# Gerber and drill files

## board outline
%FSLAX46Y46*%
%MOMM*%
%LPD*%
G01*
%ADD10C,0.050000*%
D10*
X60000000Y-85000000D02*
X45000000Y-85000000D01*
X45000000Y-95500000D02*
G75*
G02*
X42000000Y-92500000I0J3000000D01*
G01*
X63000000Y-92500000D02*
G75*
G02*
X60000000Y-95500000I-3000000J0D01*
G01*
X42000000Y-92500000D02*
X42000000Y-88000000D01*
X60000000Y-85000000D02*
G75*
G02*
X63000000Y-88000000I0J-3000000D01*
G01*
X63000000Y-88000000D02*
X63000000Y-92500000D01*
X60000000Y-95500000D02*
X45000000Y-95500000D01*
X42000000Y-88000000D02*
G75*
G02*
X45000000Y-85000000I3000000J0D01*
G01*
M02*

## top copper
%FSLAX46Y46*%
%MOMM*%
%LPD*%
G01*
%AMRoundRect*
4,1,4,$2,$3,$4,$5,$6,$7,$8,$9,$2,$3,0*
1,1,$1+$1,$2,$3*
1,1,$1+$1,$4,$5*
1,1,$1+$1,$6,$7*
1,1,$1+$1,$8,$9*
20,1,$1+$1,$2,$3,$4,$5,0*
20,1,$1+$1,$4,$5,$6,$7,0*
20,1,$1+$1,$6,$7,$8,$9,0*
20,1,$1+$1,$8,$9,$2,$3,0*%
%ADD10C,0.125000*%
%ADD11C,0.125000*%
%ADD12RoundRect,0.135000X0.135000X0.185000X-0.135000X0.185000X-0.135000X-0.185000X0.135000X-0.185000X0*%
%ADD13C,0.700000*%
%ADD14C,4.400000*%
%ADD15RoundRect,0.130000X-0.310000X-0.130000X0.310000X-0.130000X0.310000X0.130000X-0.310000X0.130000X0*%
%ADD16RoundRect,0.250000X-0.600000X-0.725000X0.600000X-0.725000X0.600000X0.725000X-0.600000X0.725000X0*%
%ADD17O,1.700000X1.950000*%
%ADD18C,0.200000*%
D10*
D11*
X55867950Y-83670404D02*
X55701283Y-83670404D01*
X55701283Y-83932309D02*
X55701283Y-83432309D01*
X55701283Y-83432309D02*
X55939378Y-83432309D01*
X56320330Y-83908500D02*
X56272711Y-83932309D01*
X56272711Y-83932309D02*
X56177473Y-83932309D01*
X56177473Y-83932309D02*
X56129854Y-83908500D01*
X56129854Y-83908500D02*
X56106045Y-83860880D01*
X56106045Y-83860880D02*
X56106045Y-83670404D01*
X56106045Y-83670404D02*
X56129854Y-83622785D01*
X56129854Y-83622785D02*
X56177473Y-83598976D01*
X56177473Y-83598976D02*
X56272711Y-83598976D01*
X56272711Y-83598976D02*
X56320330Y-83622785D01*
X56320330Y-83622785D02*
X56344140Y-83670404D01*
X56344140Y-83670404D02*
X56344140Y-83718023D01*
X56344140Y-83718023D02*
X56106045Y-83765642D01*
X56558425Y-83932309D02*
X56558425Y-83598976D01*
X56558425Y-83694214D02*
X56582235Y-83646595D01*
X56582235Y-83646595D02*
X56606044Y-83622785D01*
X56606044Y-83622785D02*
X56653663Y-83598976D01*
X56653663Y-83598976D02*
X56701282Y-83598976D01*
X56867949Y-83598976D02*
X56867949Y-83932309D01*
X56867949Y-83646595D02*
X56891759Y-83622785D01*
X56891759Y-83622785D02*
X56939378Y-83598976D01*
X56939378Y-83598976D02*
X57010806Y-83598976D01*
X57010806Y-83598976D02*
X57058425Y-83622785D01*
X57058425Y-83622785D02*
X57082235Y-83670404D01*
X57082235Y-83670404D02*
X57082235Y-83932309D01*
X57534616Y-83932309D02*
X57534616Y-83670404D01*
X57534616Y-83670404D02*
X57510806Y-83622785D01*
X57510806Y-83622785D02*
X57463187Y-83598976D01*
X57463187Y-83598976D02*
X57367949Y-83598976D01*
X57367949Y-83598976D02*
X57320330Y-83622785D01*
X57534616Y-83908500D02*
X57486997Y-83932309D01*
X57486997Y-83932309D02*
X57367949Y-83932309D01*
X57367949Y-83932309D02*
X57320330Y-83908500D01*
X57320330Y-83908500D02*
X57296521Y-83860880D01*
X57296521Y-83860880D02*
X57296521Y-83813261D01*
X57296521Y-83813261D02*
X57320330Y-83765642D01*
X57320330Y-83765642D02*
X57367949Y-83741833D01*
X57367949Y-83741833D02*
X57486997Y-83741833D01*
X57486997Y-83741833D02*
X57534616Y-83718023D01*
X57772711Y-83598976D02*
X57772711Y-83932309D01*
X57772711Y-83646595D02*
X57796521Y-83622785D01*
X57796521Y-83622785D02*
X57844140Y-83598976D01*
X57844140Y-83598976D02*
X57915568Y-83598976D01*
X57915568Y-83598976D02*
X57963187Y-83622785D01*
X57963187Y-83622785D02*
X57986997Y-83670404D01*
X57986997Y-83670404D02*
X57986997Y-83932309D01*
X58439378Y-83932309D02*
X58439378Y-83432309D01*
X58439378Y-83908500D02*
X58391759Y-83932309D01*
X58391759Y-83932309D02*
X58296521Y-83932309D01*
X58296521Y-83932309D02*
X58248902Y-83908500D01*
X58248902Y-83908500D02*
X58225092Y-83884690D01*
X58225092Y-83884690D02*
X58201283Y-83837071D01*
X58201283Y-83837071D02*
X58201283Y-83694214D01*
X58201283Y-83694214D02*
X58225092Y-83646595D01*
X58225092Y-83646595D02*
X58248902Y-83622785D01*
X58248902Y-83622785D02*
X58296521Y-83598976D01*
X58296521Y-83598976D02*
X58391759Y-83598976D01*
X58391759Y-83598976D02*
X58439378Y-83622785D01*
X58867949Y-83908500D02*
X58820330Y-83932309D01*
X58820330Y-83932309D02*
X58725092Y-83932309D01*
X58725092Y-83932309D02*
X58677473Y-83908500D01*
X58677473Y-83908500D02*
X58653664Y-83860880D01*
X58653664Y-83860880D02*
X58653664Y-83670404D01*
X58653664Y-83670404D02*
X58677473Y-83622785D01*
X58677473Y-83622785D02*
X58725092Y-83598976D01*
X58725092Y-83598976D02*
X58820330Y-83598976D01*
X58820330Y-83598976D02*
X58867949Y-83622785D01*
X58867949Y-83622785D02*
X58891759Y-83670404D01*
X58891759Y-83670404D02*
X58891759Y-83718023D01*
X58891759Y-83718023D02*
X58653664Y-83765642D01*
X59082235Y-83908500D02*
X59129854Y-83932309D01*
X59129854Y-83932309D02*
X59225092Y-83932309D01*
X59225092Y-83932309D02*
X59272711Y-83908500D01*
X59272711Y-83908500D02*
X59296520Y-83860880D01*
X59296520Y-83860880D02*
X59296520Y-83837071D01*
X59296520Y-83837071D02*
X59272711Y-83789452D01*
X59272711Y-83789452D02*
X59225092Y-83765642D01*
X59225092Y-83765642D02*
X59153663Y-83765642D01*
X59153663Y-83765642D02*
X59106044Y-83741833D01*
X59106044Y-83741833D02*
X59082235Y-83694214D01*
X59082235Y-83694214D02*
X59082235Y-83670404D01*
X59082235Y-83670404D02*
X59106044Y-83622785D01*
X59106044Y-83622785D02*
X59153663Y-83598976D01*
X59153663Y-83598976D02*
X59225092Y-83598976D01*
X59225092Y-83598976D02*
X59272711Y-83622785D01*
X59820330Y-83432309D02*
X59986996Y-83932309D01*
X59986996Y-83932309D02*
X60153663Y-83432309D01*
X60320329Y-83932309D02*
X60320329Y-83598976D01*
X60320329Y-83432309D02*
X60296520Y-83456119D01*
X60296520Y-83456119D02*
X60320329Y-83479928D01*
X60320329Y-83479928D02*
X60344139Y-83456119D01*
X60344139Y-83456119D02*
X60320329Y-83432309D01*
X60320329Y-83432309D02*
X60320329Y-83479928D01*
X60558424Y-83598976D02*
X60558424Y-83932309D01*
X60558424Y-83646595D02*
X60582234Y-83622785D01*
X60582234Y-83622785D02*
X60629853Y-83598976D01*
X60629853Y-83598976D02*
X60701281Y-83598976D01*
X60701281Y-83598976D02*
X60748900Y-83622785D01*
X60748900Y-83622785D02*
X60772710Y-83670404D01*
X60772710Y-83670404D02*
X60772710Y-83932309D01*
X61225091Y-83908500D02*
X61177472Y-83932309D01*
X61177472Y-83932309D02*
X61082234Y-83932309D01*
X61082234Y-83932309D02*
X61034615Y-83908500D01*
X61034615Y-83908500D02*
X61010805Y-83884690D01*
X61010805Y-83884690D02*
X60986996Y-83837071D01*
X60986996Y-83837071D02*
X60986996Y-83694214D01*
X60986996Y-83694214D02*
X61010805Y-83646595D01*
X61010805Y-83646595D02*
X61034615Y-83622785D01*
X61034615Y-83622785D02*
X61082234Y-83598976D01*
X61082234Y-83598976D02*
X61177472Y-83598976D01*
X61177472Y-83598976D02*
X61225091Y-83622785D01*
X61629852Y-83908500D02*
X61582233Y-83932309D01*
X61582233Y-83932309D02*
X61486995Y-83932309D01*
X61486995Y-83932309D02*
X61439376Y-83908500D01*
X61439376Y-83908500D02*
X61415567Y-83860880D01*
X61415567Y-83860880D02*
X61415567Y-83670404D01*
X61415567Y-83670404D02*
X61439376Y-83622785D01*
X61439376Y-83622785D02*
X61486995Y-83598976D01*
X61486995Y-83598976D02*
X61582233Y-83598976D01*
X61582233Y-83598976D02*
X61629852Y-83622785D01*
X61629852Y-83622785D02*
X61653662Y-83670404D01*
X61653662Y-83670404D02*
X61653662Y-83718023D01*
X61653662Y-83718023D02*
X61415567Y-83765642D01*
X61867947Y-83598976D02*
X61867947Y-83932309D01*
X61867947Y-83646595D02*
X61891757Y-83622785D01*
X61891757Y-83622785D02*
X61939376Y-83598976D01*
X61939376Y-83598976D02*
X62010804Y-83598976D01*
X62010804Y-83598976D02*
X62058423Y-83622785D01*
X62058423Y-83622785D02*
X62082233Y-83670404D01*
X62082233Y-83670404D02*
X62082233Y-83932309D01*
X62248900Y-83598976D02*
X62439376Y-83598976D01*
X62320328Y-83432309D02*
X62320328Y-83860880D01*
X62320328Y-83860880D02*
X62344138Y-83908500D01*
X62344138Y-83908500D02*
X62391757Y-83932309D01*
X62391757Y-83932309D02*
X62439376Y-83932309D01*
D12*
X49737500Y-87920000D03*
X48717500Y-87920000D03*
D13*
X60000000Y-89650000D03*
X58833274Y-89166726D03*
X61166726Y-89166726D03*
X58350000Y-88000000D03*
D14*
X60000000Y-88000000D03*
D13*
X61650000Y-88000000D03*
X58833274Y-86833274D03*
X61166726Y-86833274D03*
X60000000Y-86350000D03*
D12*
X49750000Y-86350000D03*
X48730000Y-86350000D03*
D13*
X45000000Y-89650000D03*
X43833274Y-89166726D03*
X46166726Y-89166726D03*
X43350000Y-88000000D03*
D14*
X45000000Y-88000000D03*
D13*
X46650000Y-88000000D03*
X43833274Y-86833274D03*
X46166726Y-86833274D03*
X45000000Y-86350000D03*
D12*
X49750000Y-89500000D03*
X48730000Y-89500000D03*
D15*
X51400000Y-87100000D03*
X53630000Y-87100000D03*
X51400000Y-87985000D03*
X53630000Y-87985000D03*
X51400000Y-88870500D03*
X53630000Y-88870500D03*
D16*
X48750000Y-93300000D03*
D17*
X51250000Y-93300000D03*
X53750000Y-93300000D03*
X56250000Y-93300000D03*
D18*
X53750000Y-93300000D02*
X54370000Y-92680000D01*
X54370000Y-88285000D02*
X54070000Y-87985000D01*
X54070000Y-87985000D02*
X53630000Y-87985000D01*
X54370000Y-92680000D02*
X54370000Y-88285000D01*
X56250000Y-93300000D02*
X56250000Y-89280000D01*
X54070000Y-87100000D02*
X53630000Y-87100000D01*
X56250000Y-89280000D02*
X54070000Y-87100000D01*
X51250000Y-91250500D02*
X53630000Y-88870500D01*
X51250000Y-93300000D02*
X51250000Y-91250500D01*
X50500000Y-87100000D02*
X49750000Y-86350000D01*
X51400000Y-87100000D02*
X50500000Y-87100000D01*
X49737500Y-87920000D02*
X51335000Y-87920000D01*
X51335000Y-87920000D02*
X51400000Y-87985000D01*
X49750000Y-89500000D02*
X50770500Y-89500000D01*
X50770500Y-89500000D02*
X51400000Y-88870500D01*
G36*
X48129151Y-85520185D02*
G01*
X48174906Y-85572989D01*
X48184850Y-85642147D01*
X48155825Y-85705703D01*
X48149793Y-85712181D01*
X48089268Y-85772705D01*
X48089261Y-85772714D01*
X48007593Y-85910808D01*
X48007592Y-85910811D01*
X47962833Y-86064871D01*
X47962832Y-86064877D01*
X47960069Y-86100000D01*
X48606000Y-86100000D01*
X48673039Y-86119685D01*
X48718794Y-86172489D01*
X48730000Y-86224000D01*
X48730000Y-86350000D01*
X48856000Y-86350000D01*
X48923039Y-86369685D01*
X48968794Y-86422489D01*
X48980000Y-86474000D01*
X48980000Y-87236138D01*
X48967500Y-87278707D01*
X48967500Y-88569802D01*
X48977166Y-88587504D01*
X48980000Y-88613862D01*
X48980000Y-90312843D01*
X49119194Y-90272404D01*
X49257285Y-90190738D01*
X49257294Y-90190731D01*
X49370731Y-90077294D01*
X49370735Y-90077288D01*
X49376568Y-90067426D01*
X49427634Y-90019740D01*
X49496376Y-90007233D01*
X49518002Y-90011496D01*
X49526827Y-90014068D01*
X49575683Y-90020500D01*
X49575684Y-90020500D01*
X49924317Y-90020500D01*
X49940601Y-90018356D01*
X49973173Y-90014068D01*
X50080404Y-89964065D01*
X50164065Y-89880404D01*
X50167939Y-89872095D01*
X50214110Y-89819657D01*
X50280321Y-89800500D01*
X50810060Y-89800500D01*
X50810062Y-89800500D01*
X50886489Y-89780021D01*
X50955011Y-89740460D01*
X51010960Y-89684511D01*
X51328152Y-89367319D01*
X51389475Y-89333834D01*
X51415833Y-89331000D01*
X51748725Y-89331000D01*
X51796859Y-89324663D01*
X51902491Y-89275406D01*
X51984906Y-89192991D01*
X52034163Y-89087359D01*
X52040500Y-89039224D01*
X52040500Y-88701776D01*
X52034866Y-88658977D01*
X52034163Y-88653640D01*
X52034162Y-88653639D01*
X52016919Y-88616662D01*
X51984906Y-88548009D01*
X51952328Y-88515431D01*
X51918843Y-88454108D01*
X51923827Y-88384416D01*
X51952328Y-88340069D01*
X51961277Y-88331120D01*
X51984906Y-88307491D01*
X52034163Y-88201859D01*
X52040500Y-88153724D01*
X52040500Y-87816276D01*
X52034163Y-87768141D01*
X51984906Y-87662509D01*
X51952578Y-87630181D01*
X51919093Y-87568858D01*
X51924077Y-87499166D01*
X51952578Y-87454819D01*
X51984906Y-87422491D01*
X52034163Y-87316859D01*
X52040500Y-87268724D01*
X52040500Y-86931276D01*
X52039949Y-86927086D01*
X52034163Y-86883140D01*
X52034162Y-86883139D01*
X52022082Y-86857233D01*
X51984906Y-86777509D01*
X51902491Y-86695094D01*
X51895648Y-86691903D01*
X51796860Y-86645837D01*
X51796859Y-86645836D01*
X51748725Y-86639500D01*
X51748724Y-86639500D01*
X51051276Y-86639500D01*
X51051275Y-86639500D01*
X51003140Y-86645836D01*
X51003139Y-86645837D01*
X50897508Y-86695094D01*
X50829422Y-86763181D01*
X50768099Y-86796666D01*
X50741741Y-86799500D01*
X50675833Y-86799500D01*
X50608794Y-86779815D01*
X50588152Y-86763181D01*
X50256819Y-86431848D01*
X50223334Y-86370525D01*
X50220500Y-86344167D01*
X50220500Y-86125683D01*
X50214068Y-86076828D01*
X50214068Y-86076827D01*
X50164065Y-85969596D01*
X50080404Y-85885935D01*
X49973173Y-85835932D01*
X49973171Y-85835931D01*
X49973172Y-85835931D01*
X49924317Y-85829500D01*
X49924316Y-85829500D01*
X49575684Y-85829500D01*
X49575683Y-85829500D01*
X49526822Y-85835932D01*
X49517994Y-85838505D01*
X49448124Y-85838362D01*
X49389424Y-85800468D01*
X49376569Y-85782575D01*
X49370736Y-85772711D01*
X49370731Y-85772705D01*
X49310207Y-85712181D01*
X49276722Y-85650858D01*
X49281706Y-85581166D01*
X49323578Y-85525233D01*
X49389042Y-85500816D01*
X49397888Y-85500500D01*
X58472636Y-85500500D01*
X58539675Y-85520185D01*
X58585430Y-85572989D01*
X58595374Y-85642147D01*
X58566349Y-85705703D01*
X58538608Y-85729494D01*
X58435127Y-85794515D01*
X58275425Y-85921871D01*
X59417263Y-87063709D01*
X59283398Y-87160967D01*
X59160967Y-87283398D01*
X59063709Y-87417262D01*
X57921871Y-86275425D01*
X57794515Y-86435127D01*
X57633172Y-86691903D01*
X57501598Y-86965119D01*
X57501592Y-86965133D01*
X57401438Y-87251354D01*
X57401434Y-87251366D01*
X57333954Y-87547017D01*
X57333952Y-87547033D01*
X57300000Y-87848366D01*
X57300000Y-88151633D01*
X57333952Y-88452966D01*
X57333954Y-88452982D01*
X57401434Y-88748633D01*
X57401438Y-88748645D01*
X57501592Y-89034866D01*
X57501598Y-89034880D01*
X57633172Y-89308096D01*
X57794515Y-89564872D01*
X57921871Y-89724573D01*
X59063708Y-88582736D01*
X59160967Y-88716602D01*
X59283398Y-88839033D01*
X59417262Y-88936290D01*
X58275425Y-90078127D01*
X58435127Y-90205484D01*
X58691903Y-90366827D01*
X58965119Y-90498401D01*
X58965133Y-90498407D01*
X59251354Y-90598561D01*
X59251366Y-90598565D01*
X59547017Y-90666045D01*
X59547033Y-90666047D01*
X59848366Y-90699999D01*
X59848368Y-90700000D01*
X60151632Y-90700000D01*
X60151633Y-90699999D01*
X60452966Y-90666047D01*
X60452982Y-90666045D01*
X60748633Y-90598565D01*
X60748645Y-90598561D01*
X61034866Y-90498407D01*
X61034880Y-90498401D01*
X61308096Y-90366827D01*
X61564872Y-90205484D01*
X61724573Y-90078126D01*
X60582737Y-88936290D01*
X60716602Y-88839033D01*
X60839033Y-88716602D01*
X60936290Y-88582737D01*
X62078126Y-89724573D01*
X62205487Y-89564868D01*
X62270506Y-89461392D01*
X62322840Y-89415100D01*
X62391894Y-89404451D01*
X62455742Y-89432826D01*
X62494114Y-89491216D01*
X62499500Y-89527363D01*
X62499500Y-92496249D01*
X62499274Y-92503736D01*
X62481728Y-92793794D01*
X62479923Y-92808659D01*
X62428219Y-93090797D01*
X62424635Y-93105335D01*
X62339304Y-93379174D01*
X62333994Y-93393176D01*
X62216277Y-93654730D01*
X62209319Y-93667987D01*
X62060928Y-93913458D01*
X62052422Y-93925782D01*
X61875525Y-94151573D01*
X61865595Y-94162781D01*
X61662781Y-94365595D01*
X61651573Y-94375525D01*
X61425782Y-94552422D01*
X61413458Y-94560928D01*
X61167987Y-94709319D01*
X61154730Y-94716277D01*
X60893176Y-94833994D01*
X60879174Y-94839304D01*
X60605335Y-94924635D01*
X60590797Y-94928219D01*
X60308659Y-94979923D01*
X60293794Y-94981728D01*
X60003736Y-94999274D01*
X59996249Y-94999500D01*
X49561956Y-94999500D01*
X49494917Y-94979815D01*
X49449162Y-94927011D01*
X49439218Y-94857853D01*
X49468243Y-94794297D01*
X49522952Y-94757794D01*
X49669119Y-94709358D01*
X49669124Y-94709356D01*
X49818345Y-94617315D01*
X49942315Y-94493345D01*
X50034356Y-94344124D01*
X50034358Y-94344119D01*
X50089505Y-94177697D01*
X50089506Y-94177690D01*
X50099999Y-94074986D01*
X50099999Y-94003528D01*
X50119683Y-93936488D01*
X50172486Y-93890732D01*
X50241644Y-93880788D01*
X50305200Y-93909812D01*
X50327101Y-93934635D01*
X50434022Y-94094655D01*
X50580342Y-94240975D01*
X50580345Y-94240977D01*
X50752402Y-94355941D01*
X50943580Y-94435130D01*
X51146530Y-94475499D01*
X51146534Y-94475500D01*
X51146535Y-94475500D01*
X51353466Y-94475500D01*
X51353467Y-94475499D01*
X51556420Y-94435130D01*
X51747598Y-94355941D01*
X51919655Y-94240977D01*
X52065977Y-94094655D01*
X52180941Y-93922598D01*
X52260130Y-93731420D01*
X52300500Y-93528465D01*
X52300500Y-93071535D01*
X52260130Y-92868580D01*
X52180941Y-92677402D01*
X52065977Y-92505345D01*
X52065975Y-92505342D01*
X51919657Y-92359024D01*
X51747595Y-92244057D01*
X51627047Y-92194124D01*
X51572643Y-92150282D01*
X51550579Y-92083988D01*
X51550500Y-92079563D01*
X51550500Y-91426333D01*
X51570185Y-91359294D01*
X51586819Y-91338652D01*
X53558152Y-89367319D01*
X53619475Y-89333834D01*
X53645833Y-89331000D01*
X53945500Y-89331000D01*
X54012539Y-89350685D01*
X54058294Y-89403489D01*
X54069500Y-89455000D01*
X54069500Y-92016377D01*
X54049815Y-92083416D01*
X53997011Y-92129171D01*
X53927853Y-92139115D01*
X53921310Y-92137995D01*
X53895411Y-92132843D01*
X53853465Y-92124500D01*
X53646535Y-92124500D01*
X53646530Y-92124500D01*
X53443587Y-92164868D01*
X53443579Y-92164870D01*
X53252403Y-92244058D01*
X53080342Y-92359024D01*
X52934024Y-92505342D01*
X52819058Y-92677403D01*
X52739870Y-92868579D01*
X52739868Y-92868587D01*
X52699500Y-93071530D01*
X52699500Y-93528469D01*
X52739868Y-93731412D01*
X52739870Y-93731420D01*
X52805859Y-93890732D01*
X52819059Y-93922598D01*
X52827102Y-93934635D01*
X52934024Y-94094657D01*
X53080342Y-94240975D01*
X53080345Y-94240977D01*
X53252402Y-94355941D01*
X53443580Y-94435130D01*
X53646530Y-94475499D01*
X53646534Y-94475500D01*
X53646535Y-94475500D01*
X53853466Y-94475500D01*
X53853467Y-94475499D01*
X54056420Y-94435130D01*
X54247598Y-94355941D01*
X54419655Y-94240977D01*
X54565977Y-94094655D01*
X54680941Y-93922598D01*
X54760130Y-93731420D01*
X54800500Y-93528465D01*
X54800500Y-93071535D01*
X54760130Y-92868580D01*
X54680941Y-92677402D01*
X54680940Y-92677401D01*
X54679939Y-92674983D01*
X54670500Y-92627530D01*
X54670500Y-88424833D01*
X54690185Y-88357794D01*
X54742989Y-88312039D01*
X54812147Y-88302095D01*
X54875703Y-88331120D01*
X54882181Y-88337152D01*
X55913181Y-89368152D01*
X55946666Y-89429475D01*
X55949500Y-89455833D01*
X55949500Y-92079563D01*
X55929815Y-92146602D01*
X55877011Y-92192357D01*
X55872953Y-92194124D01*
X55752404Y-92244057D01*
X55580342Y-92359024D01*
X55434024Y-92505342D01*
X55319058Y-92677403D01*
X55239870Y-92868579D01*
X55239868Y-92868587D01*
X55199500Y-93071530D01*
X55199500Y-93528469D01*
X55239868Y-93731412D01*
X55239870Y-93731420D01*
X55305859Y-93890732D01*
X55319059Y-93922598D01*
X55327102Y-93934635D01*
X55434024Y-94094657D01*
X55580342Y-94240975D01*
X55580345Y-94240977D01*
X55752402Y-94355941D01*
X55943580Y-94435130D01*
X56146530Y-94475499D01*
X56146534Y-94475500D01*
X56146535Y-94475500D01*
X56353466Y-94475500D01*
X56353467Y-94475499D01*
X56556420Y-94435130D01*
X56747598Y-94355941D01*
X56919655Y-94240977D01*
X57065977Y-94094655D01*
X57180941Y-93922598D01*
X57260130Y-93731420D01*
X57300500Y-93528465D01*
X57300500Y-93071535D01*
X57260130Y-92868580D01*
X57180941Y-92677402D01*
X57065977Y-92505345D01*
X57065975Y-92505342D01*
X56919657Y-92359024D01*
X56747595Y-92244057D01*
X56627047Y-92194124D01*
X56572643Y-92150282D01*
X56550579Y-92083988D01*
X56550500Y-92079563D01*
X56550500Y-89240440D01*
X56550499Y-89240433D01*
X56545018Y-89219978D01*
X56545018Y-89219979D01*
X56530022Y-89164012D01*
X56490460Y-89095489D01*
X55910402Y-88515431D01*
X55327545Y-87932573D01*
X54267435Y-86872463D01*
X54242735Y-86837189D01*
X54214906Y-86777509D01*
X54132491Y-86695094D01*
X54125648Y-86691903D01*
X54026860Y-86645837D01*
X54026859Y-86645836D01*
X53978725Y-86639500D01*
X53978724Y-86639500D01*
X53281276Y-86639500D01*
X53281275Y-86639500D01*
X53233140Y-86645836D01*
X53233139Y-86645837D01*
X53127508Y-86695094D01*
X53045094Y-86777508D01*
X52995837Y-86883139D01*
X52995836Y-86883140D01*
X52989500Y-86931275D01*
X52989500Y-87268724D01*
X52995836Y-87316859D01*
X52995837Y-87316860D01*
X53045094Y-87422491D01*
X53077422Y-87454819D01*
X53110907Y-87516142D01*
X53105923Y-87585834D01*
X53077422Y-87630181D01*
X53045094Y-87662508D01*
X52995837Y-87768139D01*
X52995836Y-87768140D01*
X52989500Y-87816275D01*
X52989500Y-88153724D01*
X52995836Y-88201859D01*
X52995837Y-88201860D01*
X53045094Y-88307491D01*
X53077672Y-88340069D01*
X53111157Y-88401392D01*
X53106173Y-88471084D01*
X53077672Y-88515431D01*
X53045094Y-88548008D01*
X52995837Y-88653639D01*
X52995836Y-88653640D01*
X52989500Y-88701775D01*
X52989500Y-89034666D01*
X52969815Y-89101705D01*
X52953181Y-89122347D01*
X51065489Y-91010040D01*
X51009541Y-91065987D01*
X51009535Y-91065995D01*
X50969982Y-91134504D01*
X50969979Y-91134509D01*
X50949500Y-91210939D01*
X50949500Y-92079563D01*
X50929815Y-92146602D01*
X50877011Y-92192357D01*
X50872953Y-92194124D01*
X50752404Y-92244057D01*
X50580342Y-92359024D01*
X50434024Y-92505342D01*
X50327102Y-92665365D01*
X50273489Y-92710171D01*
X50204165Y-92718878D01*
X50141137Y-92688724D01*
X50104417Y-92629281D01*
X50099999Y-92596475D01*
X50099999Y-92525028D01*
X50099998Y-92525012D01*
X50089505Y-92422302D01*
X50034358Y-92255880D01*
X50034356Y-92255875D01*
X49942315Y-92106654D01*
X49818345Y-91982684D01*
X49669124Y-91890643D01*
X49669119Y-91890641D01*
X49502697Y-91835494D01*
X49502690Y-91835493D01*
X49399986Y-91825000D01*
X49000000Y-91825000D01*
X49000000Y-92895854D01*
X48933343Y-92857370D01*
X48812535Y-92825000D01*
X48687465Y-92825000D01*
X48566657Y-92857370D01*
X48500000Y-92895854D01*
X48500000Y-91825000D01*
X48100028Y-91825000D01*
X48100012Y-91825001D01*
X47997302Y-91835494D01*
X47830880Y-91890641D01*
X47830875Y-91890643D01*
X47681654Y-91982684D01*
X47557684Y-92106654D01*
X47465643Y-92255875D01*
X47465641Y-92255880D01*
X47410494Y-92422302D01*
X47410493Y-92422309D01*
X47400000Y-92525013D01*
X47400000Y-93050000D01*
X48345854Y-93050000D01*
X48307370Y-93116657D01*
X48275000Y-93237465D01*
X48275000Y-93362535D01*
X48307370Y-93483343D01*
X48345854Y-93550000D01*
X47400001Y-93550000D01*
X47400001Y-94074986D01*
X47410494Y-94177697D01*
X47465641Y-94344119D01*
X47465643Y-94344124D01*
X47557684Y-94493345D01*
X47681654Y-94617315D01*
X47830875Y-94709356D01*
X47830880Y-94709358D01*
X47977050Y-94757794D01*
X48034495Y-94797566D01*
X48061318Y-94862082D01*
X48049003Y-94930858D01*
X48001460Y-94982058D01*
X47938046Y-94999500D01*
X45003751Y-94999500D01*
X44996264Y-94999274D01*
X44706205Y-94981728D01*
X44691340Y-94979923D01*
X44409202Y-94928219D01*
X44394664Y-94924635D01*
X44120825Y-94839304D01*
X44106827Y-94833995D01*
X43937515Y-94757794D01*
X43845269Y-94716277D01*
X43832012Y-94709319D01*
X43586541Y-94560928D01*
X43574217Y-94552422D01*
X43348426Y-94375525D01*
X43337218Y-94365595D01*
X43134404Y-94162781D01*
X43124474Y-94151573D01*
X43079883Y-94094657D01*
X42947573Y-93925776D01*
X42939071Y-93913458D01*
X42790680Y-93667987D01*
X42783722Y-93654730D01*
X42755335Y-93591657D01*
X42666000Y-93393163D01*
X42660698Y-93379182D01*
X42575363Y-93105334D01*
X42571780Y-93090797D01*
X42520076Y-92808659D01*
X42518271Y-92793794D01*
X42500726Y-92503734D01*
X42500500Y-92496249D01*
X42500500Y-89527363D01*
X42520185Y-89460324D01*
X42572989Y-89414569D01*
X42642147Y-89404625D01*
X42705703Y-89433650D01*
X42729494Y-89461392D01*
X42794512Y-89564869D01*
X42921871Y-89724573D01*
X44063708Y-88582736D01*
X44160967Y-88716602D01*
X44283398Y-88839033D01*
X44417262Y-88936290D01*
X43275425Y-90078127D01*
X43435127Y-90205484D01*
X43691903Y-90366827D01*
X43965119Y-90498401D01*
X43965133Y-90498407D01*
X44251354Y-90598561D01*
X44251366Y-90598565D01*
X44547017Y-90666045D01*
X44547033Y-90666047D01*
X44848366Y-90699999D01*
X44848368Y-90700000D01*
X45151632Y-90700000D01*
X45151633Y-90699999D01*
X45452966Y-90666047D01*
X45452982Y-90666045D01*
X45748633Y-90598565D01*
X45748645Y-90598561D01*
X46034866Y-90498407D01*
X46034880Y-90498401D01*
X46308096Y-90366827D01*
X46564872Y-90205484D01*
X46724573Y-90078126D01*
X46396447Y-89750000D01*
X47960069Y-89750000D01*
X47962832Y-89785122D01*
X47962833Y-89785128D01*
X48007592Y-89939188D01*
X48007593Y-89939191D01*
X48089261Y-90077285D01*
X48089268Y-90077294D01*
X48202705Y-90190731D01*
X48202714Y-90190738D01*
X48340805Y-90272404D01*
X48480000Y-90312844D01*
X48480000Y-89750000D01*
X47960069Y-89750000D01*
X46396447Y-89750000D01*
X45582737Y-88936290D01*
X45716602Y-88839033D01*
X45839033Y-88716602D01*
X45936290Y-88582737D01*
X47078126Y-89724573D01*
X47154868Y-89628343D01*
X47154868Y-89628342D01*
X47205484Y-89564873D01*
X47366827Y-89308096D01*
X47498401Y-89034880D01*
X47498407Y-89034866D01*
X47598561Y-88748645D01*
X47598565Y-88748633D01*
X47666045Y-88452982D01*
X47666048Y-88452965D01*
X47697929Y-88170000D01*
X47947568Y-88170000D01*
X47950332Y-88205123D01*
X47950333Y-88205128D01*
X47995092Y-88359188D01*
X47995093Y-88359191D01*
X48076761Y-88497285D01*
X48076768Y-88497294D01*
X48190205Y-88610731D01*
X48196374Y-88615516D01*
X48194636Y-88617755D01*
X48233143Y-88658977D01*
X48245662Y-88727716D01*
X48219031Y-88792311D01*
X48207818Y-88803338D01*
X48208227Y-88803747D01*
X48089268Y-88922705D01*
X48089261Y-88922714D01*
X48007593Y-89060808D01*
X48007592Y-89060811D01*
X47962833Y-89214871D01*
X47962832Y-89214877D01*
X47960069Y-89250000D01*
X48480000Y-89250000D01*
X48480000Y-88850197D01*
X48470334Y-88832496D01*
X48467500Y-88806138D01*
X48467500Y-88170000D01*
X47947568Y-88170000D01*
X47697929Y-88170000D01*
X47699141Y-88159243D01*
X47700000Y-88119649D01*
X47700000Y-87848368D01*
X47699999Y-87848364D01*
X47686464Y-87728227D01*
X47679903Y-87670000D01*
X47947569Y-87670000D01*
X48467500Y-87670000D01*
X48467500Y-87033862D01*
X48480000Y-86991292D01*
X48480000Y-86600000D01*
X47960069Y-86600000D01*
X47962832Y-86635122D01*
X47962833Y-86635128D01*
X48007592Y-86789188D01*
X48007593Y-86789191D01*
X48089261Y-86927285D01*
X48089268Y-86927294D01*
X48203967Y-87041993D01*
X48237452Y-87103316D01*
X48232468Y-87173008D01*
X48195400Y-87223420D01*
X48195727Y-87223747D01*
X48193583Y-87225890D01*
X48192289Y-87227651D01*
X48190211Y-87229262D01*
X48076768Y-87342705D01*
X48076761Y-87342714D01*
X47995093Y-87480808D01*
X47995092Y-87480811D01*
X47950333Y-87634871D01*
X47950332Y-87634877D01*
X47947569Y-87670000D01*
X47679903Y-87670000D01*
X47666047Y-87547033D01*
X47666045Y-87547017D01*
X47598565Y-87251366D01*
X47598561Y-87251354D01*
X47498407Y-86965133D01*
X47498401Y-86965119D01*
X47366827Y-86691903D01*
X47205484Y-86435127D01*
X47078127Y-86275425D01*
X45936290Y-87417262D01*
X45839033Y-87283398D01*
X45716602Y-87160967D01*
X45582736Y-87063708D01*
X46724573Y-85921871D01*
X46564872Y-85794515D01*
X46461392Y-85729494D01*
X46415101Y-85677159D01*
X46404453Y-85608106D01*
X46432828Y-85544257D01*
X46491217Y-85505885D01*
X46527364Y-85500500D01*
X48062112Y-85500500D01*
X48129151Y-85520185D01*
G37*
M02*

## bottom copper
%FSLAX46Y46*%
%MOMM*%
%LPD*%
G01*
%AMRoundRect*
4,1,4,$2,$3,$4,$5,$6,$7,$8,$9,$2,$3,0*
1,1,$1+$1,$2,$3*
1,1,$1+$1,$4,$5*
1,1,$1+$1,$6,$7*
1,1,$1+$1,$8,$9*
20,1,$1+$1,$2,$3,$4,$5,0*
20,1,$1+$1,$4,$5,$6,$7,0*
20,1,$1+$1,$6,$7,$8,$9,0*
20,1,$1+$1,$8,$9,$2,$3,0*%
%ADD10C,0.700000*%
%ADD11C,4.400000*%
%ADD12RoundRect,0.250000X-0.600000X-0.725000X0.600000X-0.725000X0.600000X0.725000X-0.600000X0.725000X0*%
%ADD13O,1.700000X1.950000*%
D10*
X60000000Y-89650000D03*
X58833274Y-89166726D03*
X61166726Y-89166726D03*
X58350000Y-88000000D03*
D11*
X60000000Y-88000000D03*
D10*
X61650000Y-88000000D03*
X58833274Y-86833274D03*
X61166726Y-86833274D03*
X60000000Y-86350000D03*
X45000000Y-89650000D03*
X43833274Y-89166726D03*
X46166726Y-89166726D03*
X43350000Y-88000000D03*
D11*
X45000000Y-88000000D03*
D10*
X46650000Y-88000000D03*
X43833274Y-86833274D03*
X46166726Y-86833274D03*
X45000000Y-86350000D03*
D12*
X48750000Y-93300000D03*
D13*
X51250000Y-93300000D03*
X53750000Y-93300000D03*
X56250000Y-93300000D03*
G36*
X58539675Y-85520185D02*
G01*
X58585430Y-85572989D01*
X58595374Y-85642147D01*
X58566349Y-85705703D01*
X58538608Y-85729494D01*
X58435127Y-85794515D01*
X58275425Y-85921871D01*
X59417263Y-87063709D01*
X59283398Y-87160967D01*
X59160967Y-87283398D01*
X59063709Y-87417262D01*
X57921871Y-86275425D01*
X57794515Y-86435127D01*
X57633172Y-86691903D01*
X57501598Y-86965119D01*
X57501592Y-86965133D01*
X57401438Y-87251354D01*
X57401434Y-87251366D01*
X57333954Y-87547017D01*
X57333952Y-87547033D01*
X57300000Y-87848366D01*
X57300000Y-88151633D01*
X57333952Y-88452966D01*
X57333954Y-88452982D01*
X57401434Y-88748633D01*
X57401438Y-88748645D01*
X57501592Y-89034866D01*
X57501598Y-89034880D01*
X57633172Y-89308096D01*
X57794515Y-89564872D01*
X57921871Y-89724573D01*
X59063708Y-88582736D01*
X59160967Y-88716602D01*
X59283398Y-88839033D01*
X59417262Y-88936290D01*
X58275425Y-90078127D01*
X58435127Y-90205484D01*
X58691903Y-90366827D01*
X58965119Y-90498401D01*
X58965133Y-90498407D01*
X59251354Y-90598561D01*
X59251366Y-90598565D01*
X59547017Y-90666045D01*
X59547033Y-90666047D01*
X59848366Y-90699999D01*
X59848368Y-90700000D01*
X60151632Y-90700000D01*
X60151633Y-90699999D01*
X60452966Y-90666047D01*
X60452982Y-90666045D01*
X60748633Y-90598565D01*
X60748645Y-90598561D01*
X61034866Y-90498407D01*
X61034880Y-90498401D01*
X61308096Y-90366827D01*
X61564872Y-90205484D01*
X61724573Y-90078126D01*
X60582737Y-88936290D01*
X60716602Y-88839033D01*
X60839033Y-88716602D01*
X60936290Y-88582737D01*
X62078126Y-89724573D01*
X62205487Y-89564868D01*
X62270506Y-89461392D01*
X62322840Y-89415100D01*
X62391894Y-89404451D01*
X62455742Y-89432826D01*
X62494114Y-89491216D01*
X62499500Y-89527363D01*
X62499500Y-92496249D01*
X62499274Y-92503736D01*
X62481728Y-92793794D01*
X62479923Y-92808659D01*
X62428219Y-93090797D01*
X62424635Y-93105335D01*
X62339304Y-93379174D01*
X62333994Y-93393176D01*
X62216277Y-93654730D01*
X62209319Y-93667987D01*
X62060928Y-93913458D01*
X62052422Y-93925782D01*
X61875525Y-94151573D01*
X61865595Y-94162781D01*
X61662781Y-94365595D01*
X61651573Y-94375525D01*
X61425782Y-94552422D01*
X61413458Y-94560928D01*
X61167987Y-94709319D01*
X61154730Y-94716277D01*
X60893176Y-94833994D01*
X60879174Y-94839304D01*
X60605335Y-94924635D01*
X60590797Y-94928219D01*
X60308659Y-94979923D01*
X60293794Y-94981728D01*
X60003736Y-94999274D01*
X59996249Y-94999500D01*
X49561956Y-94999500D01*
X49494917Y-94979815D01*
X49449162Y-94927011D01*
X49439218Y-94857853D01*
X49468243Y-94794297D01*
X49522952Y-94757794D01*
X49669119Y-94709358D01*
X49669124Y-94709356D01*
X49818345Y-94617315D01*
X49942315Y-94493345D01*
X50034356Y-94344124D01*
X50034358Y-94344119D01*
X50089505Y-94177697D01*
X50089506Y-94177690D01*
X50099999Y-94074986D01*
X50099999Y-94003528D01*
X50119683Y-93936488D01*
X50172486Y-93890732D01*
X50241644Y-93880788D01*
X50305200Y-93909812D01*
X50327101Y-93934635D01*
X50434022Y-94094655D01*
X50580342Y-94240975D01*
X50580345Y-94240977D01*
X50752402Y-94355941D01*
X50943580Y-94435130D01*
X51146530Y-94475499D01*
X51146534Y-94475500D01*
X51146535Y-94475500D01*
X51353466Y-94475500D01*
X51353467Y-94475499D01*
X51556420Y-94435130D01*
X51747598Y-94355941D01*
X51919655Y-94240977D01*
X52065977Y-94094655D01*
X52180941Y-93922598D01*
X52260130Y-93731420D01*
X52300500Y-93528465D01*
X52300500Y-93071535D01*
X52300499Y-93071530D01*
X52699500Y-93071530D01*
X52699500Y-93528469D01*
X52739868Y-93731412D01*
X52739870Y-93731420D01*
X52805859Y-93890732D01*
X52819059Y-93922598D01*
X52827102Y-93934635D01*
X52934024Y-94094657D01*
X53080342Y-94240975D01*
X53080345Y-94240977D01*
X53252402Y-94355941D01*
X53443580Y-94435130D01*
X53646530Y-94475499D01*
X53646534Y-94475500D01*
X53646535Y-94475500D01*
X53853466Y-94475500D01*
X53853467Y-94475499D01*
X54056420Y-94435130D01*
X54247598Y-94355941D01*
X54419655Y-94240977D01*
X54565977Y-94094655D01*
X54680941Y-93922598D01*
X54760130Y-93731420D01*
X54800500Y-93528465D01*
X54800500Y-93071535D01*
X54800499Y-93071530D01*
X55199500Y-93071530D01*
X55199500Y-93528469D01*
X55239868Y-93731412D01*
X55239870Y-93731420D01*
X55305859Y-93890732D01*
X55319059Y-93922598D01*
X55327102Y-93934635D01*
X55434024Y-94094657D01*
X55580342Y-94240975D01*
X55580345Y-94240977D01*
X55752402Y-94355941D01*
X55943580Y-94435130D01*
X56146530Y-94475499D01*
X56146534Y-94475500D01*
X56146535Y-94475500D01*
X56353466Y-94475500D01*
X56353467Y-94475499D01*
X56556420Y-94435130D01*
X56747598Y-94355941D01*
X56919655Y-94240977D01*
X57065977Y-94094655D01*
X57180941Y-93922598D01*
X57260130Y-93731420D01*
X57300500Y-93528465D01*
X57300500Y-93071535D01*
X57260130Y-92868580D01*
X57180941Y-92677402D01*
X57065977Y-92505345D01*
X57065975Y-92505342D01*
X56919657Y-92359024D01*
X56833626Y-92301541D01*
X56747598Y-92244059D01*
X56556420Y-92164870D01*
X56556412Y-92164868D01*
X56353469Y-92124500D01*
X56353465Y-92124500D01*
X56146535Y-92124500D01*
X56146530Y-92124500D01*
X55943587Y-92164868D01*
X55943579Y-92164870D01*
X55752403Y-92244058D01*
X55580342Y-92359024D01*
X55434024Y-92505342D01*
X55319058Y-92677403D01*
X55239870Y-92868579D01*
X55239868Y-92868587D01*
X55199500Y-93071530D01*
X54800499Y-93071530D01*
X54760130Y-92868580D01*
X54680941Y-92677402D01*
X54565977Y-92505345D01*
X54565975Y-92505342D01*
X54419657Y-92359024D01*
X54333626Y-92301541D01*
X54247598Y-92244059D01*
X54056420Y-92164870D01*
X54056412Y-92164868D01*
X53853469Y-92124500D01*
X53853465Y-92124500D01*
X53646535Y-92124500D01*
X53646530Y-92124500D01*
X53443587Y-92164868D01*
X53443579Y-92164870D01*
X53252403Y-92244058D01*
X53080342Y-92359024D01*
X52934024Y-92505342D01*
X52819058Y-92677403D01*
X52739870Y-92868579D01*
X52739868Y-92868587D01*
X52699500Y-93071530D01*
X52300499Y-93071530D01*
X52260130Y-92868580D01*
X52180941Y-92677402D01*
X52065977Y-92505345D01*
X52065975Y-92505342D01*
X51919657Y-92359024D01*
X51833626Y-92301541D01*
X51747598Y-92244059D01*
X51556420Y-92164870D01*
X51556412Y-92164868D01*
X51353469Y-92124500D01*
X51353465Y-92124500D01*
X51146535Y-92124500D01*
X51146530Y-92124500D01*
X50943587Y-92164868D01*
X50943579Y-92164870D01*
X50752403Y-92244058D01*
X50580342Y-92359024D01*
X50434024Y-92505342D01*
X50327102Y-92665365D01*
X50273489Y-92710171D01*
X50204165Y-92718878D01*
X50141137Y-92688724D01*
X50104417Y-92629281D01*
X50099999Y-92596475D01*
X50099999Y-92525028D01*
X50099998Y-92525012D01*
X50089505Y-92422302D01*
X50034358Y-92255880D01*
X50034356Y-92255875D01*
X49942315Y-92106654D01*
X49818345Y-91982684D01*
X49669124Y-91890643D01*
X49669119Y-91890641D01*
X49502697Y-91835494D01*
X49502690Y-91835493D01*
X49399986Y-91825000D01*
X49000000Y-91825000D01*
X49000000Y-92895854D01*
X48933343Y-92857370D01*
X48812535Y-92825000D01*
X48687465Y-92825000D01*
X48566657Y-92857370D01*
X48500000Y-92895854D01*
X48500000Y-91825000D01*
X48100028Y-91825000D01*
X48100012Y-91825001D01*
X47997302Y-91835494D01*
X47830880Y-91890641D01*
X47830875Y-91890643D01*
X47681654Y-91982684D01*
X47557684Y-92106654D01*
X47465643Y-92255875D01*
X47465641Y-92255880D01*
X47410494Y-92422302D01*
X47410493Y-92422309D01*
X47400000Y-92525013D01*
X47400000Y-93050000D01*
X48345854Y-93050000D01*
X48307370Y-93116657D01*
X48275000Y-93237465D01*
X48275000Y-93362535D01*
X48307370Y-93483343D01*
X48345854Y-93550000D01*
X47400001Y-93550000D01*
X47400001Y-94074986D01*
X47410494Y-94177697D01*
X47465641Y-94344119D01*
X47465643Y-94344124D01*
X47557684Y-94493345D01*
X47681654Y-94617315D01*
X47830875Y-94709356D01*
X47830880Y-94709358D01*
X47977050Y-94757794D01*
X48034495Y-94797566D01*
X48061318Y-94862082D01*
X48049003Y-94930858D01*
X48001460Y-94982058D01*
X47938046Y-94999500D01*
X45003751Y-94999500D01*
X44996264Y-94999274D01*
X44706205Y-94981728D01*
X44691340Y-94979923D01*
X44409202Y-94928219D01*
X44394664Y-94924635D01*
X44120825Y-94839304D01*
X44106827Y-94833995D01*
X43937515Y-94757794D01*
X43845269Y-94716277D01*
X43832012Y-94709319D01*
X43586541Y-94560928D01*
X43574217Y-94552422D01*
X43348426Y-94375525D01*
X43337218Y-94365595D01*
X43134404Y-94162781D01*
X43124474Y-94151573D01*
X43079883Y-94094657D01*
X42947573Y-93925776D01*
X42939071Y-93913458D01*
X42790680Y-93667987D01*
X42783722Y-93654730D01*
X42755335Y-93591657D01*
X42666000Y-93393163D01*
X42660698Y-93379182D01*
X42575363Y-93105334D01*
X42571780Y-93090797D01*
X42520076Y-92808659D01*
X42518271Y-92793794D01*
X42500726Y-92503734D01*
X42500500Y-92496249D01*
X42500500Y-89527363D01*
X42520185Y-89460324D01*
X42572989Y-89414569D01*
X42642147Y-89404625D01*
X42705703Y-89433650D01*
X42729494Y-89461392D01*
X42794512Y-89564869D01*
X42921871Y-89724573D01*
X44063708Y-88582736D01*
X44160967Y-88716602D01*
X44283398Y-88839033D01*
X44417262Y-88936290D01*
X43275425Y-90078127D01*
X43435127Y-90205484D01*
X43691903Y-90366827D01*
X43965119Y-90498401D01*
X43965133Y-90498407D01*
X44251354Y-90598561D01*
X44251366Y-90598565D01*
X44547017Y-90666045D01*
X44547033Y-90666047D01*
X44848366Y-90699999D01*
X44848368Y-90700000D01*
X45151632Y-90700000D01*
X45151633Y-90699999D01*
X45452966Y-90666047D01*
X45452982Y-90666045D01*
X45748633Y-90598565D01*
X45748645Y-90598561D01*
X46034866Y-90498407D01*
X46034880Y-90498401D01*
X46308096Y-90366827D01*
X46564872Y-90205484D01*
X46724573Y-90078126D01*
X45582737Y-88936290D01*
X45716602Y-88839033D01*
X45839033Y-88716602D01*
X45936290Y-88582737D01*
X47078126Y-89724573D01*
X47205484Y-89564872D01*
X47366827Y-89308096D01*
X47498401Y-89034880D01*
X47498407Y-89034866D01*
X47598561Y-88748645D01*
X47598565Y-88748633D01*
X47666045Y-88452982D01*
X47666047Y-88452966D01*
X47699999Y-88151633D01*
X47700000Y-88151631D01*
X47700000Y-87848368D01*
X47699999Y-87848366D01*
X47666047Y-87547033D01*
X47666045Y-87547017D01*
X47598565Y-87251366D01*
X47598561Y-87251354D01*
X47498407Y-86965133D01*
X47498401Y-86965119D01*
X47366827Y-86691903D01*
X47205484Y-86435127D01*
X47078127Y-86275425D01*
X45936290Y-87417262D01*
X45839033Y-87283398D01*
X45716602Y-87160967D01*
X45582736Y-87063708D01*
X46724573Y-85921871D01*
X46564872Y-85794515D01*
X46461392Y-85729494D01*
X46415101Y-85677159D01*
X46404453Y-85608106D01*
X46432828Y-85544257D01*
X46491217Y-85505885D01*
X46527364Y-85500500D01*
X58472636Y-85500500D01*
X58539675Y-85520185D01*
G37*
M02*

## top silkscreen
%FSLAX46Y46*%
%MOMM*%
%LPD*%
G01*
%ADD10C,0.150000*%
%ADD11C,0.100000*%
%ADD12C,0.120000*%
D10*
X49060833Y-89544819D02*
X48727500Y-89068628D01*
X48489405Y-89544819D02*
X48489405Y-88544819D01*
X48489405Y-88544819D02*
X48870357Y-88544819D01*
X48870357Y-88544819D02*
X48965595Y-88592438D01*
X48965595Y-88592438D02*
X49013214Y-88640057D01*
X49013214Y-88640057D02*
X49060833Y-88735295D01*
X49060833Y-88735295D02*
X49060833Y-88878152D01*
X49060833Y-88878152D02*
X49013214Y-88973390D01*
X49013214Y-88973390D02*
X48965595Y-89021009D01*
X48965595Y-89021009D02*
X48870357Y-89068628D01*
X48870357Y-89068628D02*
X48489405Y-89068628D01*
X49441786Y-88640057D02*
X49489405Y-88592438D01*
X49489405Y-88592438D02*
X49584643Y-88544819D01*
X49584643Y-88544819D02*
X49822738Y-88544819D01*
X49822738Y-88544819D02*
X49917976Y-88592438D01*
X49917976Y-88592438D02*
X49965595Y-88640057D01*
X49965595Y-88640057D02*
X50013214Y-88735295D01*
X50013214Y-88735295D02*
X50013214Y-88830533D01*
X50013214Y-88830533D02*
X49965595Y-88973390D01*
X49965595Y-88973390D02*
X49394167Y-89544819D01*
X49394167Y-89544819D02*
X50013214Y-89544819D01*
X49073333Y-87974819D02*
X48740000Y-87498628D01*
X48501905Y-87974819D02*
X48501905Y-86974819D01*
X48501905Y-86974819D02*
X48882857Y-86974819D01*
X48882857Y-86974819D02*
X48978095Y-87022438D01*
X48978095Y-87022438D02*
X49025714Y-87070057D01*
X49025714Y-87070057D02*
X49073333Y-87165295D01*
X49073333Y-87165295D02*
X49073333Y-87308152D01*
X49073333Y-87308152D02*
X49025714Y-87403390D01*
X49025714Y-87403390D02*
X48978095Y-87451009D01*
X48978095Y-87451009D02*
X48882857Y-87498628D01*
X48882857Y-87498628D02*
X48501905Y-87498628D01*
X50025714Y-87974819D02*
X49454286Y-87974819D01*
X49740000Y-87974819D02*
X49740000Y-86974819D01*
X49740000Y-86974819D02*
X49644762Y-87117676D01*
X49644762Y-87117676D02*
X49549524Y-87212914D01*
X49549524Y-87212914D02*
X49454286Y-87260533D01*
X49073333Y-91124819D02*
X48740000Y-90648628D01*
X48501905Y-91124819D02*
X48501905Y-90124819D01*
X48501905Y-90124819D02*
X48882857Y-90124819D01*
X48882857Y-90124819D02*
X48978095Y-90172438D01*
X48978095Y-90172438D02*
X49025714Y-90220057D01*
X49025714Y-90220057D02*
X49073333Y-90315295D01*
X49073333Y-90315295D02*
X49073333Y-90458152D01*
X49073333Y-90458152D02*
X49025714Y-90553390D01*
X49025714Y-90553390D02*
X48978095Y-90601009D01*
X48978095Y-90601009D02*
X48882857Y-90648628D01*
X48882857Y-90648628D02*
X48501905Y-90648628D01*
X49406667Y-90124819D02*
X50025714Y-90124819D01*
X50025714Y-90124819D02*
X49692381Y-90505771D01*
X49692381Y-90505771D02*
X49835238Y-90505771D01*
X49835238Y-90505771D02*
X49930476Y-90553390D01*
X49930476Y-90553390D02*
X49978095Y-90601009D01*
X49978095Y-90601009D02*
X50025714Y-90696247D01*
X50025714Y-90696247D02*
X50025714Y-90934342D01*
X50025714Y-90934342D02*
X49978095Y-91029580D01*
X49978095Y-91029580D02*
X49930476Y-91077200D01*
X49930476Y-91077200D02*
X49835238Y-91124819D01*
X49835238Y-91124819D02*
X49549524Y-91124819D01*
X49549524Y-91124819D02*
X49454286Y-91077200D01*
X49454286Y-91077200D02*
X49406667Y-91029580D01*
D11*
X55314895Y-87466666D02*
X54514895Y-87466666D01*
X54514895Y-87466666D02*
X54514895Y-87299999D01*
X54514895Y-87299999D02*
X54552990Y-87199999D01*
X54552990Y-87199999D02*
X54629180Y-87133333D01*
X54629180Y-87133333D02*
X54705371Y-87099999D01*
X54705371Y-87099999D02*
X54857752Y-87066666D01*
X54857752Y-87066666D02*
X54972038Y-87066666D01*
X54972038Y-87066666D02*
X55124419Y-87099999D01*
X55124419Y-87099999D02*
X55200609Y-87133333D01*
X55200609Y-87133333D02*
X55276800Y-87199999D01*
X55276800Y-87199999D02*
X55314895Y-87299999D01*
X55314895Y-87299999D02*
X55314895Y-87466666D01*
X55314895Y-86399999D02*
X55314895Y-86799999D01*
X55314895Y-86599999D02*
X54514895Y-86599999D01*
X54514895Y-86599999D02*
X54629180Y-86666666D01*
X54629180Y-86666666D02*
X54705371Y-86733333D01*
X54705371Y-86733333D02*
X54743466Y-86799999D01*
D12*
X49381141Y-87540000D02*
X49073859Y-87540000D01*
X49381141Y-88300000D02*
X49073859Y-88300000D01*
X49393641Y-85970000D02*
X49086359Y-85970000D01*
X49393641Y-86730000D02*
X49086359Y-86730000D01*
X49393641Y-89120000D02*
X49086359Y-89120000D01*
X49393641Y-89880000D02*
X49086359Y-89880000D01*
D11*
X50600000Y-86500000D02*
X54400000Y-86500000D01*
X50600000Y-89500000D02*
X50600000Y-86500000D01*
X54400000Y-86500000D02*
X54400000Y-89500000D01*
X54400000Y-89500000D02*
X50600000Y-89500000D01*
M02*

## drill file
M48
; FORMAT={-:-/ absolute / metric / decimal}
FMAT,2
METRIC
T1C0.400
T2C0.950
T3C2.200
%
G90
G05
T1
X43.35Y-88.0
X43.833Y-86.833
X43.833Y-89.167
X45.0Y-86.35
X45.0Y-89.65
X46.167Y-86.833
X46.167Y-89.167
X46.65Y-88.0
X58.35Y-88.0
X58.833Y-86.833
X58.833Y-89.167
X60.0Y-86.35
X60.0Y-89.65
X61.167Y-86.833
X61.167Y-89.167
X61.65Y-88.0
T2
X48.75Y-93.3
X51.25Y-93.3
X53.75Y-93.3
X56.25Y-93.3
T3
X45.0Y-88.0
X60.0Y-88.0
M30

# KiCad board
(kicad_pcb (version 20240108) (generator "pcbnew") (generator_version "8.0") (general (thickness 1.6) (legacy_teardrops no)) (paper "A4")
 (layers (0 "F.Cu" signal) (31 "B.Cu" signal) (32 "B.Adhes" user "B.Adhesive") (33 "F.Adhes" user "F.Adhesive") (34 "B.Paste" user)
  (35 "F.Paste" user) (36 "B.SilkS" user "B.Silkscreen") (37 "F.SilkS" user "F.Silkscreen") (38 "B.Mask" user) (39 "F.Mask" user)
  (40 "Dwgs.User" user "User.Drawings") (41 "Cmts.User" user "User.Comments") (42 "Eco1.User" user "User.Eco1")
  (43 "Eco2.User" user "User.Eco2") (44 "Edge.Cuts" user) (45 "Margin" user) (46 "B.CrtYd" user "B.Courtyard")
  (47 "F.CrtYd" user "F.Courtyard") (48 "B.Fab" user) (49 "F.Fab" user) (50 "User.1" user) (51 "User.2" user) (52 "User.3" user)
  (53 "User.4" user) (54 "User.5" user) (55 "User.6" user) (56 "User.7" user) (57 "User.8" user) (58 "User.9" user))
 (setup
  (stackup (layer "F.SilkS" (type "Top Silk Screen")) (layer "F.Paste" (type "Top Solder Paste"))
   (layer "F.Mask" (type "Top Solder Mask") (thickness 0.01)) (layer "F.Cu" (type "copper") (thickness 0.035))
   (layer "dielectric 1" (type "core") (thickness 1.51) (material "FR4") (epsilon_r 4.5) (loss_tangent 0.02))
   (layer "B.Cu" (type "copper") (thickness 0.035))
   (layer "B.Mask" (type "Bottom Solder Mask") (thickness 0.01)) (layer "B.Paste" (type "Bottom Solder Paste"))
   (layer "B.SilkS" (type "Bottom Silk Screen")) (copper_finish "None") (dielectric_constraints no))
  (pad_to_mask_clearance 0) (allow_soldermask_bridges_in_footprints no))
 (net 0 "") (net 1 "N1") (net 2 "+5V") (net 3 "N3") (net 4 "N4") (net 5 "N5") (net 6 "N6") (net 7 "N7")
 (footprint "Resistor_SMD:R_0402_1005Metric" (layer "F.Cu") (at 49.2275 87.92 180)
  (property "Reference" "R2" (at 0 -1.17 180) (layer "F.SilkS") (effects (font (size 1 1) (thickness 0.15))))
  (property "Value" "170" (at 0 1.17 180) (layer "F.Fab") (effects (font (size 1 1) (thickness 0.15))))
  (fp_line (start -0.153641 0.38) (end 0.153641 0.38) (stroke (width 0.12) (type solid)) (layer "F.SilkS"))
  (fp_line (start -0.153641 -0.38) (end 0.153641 -0.38) (stroke (width 0.12) (type solid)) (layer "F.SilkS"))
  (pad "1" smd roundrect (at -0.51 0 180) (size 0.54 0.64) (layers "F.Cu" "F.Paste" "F.Mask") (roundrect_rratio 0.25) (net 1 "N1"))
  (pad "2" smd roundrect (at 0.51 0 180) (size 0.54 0.64) (layers "F.Cu" "F.Paste" "F.Mask") (roundrect_rratio 0.25) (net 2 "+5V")))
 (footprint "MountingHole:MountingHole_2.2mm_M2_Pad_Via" (layer "F.Cu") (at 60 88 90)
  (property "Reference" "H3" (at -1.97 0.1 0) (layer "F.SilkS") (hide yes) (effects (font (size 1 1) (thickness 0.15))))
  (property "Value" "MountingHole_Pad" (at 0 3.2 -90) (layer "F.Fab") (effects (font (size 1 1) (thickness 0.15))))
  (pad "1" thru_hole circle (at -1.65 0 90) (size 0.7 0.7) (drill 0.4) (layers "*.Cu" "*.Mask") (remove_unused_layers no) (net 2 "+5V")
   (zone_connect 2))
  (pad "1" thru_hole circle (at -1.166726 -1.166726 90) (size 0.7 0.7) (drill 0.4) (layers "*.Cu" "*.Mask") (remove_unused_layers no)
   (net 2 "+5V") (zone_connect 2))
  (pad "1" thru_hole circle (at -1.166726 1.166726 90) (size 0.7 0.7) (drill 0.4) (layers "*.Cu" "*.Mask") (remove_unused_layers no)
   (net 2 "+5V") (zone_connect 2))
  (pad "1" thru_hole circle (at 0 -1.65 90) (size 0.7 0.7) (drill 0.4) (layers "*.Cu" "*.Mask") (remove_unused_layers no) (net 2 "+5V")
   (zone_connect 2))
  (pad "1" thru_hole circle (at 0 0 90) (size 4.4 4.4) (drill 2.2) (layers "*.Cu" "*.Mask") (remove_unused_layers no) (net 2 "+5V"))
  (pad "1" thru_hole circle (at 0 1.65 90) (size 0.7 0.7) (drill 0.4) (layers "*.Cu" "*.Mask") (remove_unused_layers no) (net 2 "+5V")
   (zone_connect 2))
  (pad "1" thru_hole circle (at 1.166726 -1.166726 90) (size 0.7 0.7) (drill 0.4) (layers "*.Cu" "*.Mask") (remove_unused_layers no)
   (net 2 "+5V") (zone_connect 2))
  (pad "1" thru_hole circle (at 1.166726 1.166726 90) (size 0.7 0.7) (drill 0.4) (layers "*.Cu" "*.Mask") (remove_unused_layers no)
   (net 2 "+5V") (zone_connect 2))
  (pad "1" thru_hole circle (at 1.65 0 90) (size 0.7 0.7) (drill 0.4) (layers "*.Cu" "*.Mask") (remove_unused_layers no) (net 2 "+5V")
   (zone_connect 2)))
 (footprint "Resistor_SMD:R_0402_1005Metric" (layer "F.Cu") (at 49.24 86.35 180)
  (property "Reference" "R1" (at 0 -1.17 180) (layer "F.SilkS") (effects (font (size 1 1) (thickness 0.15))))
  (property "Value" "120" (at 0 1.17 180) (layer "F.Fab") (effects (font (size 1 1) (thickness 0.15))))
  (fp_line (start -0.153641 0.38) (end 0.153641 0.38) (stroke (width 0.12) (type solid)) (layer "F.SilkS"))
  (fp_line (start -0.153641 -0.38) (end 0.153641 -0.38) (stroke (width 0.12) (type solid)) (layer "F.SilkS"))
  (pad "1" smd roundrect (at -0.51 0 180) (size 0.54 0.64) (layers "F.Cu" "F.Paste" "F.Mask") (roundrect_rratio 0.25) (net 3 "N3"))
  (pad "2" smd roundrect (at 0.51 0 180) (size 0.54 0.64) (layers "F.Cu" "F.Paste" "F.Mask") (roundrect_rratio 0.25) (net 2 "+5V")))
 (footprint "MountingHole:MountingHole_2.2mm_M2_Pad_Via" (layer "F.Cu") (at 45 88 90)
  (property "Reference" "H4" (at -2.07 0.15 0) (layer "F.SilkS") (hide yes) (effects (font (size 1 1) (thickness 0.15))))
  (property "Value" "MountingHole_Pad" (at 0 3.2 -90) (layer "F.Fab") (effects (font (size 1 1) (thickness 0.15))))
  (pad "1" thru_hole circle (at -1.65 0 90) (size 0.7 0.7) (drill 0.4) (layers "*.Cu" "*.Mask") (remove_unused_layers no) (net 2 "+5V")
   (zone_connect 2))
  (pad "1" thru_hole circle (at -1.166726 -1.166726 90) (size 0.7 0.7) (drill 0.4) (layers "*.Cu" "*.Mask") (remove_unused_layers no)
   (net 2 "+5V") (zone_connect 2))
  (pad "1" thru_hole circle (at -1.166726 1.166726 90) (size 0.7 0.7) (drill 0.4) (layers "*.Cu" "*.Mask") (remove_unused_layers no)
   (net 2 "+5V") (zone_connect 2))
  (pad "1" thru_hole circle (at 0 -1.65 90) (size 0.7 0.7) (drill 0.4) (layers "*.Cu" "*.Mask") (remove_unused_layers no) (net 2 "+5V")
   (zone_connect 2))
  (pad "1" thru_hole circle (at 0 0 90) (size 4.4 4.4) (drill 2.2) (layers "*.Cu" "*.Mask") (remove_unused_layers no) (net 2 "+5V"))
  (pad "1" thru_hole circle (at 0 1.65 90) (size 0.7 0.7) (drill 0.4) (layers "*.Cu" "*.Mask") (remove_unused_layers no) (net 2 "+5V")
   (zone_connect 2))
  (pad "1" thru_hole circle (at 1.166726 -1.166726 90) (size 0.7 0.7) (drill 0.4) (layers "*.Cu" "*.Mask") (remove_unused_layers no)
   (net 2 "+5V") (zone_connect 2))
  (pad "1" thru_hole circle (at 1.166726 1.166726 90) (size 0.7 0.7) (drill 0.4) (layers "*.Cu" "*.Mask") (remove_unused_layers no)
   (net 2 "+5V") (zone_connect 2))
  (pad "1" thru_hole circle (at 1.65 0 90) (size 0.7 0.7) (drill 0.4) (layers "*.Cu" "*.Mask") (remove_unused_layers no) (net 2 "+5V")
   (zone_connect 2)))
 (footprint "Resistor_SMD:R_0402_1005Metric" (layer "F.Cu") (at 49.24 89.5 180)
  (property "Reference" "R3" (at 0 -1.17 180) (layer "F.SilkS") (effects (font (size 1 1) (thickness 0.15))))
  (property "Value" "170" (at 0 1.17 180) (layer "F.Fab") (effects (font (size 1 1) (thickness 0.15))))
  (fp_line (start -0.153641 0.38) (end 0.153641 0.38) (stroke (width 0.12) (type solid)) (layer "F.SilkS"))
  (fp_line (start -0.153641 -0.38) (end 0.153641 -0.38) (stroke (width 0.12) (type solid)) (layer "F.SilkS"))
  (pad "1" smd roundrect (at -0.51 0 180) (size 0.54 0.64) (layers "F.Cu" "F.Paste" "F.Mask") (roundrect_rratio 0.25) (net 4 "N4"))
  (pad "2" smd roundrect (at 0.51 0 180) (size 0.54 0.64) (layers "F.Cu" "F.Paste" "F.Mask") (roundrect_rratio 0.25) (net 2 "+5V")))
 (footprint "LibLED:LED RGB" (layer "F.Cu") (at 52.5 88)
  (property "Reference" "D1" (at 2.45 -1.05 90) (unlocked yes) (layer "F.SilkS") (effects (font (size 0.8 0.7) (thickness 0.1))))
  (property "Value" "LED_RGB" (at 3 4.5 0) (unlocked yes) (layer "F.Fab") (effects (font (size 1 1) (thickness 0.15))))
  (fp_line (start -1.9 -1.5) (end 1.9 -1.5) (stroke (width 0.1) (type default)) (layer "F.SilkS"))
  (fp_line (start -1.9 1.5) (end -1.9 -1.5) (stroke (width 0.1) (type default)) (layer "F.SilkS"))
  (fp_line (start 1.9 -1.5) (end 1.9 1.5) (stroke (width 0.1) (type default)) (layer "F.SilkS"))
  (fp_line (start 1.9 1.5) (end -1.9 1.5) (stroke (width 0.1) (type default)) (layer "F.SilkS"))
  (pad "1" smd roundrect (at -1.1 -0.9) (size 0.88 0.52) (layers "F.Cu" "F.Paste" "F.Mask") (roundrect_rratio 0.25) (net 3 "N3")
   (thermal_bridge_angle 45))
  (pad "2" smd roundrect (at 1.13 -0.9) (size 0.88 0.52) (layers "F.Cu" "F.Paste" "F.Mask") (roundrect_rratio 0.25) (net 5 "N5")
   (thermal_bridge_angle 45))
  (pad "3" smd roundrect (at -1.1 -0.015) (size 0.88 0.52) (layers "F.Cu" "F.Paste" "F.Mask") (roundrect_rratio 0.25) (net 1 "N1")
   (thermal_bridge_angle 45))
  (pad "4" smd roundrect (at 1.13 -0.015) (size 0.88 0.52) (layers "F.Cu" "F.Paste" "F.Mask") (roundrect_rratio 0.25) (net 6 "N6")
   (thermal_bridge_angle 45))
  (pad "5" smd roundrect (at -1.1 0.8705) (size 0.88 0.52) (layers "F.Cu" "F.Paste" "F.Mask") (roundrect_rratio 0.25) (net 4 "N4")
   (thermal_bridge_angle 45))
  (pad "6" smd roundrect (at 1.13 0.8705) (size 0.88 0.52) (layers "F.Cu" "F.Paste" "F.Mask") (roundrect_rratio 0.25) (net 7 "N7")
   (thermal_bridge_angle 45)))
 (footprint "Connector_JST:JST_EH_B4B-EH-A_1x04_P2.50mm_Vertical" (layer "B.Cu") (at 48.75 93.3)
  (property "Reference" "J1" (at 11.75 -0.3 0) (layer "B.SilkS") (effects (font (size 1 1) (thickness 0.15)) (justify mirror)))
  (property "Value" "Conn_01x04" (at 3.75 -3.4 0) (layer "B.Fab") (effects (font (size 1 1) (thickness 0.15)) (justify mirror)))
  (pad "1" thru_hole roundrect (at 0 0) (size 1.7 1.95) (drill 0.95) (layers "*.Cu" "*.Mask") (remove_unused_layers no)
   (roundrect_rratio 0.147059) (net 2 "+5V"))
  (pad "2" thru_hole oval (at 2.5 0) (size 1.7 1.95) (drill 0.95) (layers "*.Cu" "*.Mask") (remove_unused_layers no) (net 7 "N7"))
  (pad "3" thru_hole oval (at 5 0) (size 1.7 1.95) (drill 0.95) (layers "*.Cu" "*.Mask") (remove_unused_layers no) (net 6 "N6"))
  (pad "4" thru_hole oval (at 7.5 0) (size 1.7 1.95) (drill 0.95) (layers "*.Cu" "*.Mask") (remove_unused_layers no) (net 5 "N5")))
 (gr_line (start 60 85) (end 45 85) (stroke (width 0.05) (type default)) (layer "Edge.Cuts"))
 (gr_arc (start 45 95.5) (mid 42.87868 94.62132) (end 42 92.5) (stroke (width 0.05) (type default)) (layer "Edge.Cuts"))
 (gr_arc (start 63 92.5) (mid 62.12132 94.62132) (end 60 95.5) (stroke (width 0.05) (type default)) (layer "Edge.Cuts"))
 (gr_line (start 42 92.5) (end 42 88) (stroke (width 0.05) (type default)) (layer "Edge.Cuts"))
 (gr_arc (start 60 85) (mid 62.12132 85.87868) (end 63 88) (stroke (width 0.05) (type default)) (layer "Edge.Cuts"))
 (gr_line (start 63 88) (end 63 92.5) (stroke (width 0.05) (type default)) (layer "Edge.Cuts"))
 (gr_line (start 60 95.5) (end 45 95.5) (stroke (width 0.05) (type default)) (layer "Edge.Cuts"))
 (gr_arc (start 42 88) (mid 42.87868 85.87868) (end 45 85) (stroke (width 0.05) (type default)) (layer "Edge.Cuts"))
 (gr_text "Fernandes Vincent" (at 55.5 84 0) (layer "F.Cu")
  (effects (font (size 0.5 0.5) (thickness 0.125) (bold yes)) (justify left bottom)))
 (segment (start 53.75 93.3) (end 54.37 92.68) (width 0.2) (layer "F.Cu") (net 6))
 (segment (start 54.37 88.285) (end 54.07 87.985) (width 0.2) (layer "F.Cu") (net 6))
 (segment (start 54.07 87.985) (end 53.63 87.985) (width 0.2) (layer "F.Cu") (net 6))
 (segment (start 54.37 92.68) (end 54.37 88.285) (width 0.2) (layer "F.Cu") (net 6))
 (segment (start 56.25 93.3) (end 56.25 89.28) (width 0.2) (layer "F.Cu") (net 5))
 (segment (start 54.07 87.1) (end 53.63 87.1) (width 0.2) (layer "F.Cu") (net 5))
 (segment (start 56.25 89.28) (end 54.07 87.1) (width 0.2) (layer "F.Cu") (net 5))
 (segment (start 51.25 91.2505) (end 53.63 88.8705) (width 0.2) (layer "F.Cu") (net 7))
 (segment (start 51.25 93.3) (end 51.25 91.2505) (width 0.2) (layer "F.Cu") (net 7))
 (segment (start 50.5 87.1) (end 49.75 86.35) (width 0.2) (layer "F.Cu") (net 3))
 (segment (start 51.4 87.1) (end 50.5 87.1) (width 0.2) (layer "F.Cu") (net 3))
 (segment (start 49.7375 87.92) (end 51.335 87.92) (width 0.2) (layer "F.Cu") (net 1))
 (segment (start 51.335 87.92) (end 51.4 87.985) (width 0.2) (layer "F.Cu") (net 1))
 (segment (start 49.75 89.5) (end 50.7705 89.5) (width 0.2) (layer "F.Cu") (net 4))
 (segment (start 50.7705 89.5) (end 51.4 88.8705) (width 0.2) (layer "F.Cu") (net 4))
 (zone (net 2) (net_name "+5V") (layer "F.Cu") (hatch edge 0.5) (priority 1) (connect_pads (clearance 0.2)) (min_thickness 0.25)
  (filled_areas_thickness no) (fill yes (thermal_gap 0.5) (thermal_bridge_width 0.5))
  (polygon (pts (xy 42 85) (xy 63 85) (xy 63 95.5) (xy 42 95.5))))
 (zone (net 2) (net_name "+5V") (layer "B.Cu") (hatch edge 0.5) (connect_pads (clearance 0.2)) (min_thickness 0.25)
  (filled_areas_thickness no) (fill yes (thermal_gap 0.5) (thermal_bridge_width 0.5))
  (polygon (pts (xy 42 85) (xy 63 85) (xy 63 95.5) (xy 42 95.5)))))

